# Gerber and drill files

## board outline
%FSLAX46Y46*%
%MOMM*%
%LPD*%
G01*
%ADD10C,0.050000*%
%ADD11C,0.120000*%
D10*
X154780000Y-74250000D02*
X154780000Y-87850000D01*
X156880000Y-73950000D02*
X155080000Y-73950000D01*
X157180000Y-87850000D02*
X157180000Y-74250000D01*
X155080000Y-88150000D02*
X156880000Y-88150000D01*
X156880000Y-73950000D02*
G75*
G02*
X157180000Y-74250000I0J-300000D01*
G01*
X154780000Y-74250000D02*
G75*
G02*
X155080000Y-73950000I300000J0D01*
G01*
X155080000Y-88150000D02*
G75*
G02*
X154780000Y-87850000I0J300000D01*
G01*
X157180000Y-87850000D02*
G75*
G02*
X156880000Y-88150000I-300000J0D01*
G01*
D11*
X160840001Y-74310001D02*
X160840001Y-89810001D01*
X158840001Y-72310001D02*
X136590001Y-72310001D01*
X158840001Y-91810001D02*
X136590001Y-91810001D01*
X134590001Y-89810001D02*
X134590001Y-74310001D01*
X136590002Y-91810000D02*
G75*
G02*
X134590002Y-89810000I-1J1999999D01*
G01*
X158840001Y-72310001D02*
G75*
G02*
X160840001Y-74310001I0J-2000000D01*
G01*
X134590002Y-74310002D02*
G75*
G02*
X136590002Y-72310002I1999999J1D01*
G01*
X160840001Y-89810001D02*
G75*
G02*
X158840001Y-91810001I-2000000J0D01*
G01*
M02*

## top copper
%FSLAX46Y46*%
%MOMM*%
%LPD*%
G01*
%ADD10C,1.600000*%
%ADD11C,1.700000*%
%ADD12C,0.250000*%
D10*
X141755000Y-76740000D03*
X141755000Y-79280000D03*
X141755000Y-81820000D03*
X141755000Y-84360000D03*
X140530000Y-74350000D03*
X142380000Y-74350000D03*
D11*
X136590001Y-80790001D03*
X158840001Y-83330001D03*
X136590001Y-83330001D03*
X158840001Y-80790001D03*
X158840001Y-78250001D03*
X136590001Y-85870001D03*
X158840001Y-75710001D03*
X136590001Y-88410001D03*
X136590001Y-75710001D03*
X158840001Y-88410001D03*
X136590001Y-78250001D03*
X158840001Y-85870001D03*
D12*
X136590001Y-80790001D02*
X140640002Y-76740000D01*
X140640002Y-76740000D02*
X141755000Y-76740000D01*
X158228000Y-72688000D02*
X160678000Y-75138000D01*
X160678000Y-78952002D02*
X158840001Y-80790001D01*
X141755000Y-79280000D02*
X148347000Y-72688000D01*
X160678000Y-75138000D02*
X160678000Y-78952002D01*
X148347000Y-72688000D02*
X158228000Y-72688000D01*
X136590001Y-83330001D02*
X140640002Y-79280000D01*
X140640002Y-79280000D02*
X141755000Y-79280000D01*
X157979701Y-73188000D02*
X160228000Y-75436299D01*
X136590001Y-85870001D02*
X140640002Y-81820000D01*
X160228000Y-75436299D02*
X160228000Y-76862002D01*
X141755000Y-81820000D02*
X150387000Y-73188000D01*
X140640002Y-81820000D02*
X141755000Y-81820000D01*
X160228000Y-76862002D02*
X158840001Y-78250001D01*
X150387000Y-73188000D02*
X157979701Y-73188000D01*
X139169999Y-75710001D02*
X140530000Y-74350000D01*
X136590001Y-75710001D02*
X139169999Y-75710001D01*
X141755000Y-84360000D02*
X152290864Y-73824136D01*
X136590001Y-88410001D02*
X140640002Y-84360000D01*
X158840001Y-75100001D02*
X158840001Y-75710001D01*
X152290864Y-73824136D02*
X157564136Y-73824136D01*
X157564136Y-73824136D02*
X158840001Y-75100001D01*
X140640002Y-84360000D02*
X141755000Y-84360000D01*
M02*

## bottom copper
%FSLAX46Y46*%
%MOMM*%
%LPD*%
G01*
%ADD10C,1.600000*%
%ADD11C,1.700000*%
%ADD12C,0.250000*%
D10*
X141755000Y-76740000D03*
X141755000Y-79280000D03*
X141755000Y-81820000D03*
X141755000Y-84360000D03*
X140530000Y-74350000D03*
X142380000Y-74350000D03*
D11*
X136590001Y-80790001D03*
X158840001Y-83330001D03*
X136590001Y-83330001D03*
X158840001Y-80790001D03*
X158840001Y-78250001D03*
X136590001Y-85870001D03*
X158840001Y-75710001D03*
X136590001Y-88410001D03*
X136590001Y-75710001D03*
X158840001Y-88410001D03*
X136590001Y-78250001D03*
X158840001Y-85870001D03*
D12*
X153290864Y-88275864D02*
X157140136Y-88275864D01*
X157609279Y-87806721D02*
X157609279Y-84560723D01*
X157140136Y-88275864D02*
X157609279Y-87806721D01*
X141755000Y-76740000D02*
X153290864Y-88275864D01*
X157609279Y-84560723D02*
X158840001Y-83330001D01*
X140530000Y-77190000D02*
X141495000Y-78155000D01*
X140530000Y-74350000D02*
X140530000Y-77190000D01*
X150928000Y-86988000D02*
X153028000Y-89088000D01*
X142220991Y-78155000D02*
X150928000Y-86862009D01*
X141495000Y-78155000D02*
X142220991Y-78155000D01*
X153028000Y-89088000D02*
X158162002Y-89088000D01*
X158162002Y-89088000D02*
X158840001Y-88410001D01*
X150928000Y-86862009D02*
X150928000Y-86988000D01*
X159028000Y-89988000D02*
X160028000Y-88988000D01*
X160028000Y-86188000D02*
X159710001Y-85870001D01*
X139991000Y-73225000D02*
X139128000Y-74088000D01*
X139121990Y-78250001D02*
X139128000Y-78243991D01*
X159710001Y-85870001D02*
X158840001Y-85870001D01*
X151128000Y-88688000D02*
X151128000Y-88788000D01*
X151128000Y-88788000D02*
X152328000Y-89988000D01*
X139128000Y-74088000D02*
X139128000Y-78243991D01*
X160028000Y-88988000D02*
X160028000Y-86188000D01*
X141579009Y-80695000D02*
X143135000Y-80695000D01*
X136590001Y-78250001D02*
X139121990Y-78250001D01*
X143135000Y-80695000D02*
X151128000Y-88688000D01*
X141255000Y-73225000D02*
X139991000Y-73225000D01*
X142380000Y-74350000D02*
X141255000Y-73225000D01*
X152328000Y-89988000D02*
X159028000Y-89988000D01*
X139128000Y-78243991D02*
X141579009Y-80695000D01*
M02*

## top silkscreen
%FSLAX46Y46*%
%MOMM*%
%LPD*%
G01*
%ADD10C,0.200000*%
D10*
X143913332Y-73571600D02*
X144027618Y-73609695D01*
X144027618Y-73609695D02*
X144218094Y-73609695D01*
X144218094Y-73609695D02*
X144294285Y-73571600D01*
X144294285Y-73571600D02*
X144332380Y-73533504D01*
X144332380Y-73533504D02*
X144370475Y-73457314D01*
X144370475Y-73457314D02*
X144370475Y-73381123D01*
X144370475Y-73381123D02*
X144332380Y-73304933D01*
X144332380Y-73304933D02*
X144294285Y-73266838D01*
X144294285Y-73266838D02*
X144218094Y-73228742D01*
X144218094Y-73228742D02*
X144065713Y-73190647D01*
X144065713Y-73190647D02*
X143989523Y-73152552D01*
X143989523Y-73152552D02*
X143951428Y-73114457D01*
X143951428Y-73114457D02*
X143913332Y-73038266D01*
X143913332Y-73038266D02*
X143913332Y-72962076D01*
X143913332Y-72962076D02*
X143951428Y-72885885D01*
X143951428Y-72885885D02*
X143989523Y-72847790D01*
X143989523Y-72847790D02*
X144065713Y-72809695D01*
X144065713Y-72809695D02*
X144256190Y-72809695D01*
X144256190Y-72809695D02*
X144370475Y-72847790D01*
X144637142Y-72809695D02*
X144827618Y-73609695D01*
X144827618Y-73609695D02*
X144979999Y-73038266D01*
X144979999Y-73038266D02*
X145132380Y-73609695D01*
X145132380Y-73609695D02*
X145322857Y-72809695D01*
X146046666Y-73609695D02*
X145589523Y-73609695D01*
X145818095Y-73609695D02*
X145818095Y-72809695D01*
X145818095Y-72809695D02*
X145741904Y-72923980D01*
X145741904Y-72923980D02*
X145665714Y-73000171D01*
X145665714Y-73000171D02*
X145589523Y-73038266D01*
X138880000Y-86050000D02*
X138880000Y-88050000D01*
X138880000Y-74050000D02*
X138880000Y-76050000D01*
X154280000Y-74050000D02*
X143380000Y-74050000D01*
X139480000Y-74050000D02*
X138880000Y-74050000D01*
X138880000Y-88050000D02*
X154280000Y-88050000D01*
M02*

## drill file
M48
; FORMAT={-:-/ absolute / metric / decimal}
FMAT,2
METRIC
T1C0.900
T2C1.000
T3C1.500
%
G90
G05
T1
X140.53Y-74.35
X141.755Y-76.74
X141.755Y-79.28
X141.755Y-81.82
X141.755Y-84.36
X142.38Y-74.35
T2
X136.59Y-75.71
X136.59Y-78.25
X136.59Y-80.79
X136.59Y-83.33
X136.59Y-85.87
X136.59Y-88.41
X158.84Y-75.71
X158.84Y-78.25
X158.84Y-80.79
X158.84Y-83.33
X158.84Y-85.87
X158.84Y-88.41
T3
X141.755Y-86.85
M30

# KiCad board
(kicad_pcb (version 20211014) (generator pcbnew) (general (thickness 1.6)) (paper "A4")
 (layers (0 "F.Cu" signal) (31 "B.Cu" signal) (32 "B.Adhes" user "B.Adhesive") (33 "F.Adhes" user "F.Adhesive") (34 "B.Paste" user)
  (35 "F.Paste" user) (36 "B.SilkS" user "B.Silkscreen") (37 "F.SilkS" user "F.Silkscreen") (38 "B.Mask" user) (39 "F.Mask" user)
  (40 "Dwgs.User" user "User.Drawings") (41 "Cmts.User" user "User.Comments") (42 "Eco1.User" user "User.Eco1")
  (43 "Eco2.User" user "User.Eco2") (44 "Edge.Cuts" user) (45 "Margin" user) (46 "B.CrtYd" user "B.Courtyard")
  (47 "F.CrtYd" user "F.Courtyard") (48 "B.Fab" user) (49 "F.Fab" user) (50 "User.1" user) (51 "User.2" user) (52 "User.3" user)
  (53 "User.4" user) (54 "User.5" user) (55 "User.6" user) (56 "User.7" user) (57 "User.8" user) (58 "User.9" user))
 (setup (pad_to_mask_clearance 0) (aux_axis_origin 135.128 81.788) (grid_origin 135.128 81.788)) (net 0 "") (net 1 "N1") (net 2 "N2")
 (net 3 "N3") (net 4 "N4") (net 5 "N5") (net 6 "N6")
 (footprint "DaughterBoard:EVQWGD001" (layer "F.Cu") (at 147.38 80.55)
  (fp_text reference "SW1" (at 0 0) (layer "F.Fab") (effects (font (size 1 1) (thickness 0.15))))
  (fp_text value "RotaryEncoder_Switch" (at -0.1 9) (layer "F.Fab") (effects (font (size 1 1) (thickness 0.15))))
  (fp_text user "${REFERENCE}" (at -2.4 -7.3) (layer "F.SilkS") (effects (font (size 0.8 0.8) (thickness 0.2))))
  (fp_line (start -8.5 5.5) (end -8.5 7.5) (layer "F.SilkS") (width 0.2))
  (fp_line (start -8.5 -6.5) (end -8.5 -4.5) (layer "F.SilkS") (width 0.2))
  (fp_line (start 6.9 -6.5) (end -4 -6.5) (layer "F.SilkS") (width 0.2))
  (fp_line (start -7.9 -6.5) (end -8.5 -6.5) (layer "F.SilkS") (width 0.2))
  (fp_line (start -8.5 7.5) (end 6.9 7.5) (layer "F.SilkS") (width 0.2))
  (fp_line (start 7.4 -6.3) (end 7.4 7.3) (layer "Edge.Cuts") (width 0.05))
  (fp_line (start 9.5 -6.6) (end 7.7 -6.6) (layer "Edge.Cuts") (width 0.05))
  (fp_line (start 9.8 7.3) (end 9.8 -6.3) (layer "Edge.Cuts") (width 0.05))
  (fp_line (start 7.7 7.6) (end 9.5 7.6) (layer "Edge.Cuts") (width 0.05))
  (fp_arc (start 9.5 -6.6) (mid 9.712132 -6.512132) (end 9.8 -6.3) (layer "Edge.Cuts") (width 0.05))
  (fp_arc (start 7.4 -6.3) (mid 7.487868 -6.512132) (end 7.7 -6.6) (layer "Edge.Cuts") (width 0.05))
  (fp_arc (start 7.7 7.6) (mid 7.487868 7.512132) (end 7.4 7.3) (layer "Edge.Cuts") (width 0.05))
  (fp_arc (start 9.8 7.3) (mid 9.712132 7.512132) (end 9.5 7.6) (layer "Edge.Cuts") (width 0.05))
  (pad "" np_thru_hole circle (at -5.625 6.3) (size 1.5 1.5) (drill 1.5) (layers *.Cu *.Mask))
  (pad "A" thru_hole circle (at -5.625 -3.81) (size 1.6 1.6) (drill 0.9) (layers *.Cu *.Mask) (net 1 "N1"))
  (pad "B" thru_hole circle (at -5.625 -1.27) (size 1.6 1.6) (drill 0.9) (layers *.Cu *.Mask) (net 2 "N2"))
  (pad "C" thru_hole circle (at -5.625 1.27) (size 1.6 1.6) (drill 0.9) (layers *.Cu *.Mask) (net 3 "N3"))
  (pad "D" thru_hole circle (at -5.625 3.81) (size 1.6 1.6) (drill 0.9) (layers *.Cu *.Mask) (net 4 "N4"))
  (pad "S1" thru_hole circle (at -6.85 -6.2) (size 1.6 1.6) (drill 0.9) (layers *.Cu *.Mask) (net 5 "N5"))
  (pad "S2" thru_hole circle (at -5 -6.2) (size 1.6 1.6) (drill 0.9) (layers *.Cu *.Mask) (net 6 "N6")))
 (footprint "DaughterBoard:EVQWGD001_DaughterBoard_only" (layer "F.Cu") (at 147.840001 82.060001)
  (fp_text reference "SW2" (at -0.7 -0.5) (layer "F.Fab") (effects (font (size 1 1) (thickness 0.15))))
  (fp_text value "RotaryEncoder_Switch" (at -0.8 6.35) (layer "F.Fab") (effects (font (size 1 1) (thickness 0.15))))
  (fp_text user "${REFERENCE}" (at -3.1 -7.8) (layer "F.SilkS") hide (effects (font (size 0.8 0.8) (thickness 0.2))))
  (fp_line (start 13 -7.75) (end 13 7.75) (layer "Edge.Cuts") (width 0.12))
  (fp_line (start 11 -9.75) (end -11.25 -9.75) (layer "Edge.Cuts") (width 0.12))
  (fp_line (start 11 9.75) (end -11.25 9.75) (layer "Edge.Cuts") (width 0.12))
  (fp_line (start -13.25 7.75) (end -13.25 -7.75) (layer "Edge.Cuts") (width 0.12))
  (fp_arc (start -11.249999 9.749999) (mid -12.664213 9.164213) (end -13.249999 7.749999) (layer "Edge.Cuts") (width 0.12))
  (fp_arc (start 11 -9.75) (mid 12.414214 -9.164214) (end 13 -7.75) (layer "Edge.Cuts") (width 0.12))
  (fp_arc (start -13.249999 -7.749999) (mid -12.664213 -9.164213) (end -11.249999 -9.749999) (layer "Edge.Cuts") (width 0.12))
  (fp_arc (start 13 7.75) (mid 12.414214 9.164214) (end 11 9.75) (layer "Edge.Cuts") (width 0.12))
  (pad "A" thru_hole circle (at -11.25 -1.27) (size 1.7 1.7) (drill 1) (layers *.Cu *.Mask) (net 1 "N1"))
  (pad "A" thru_hole circle (at 11 1.27 180) (size 1.7 1.7) (drill 1) (layers *.Cu *.Mask) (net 1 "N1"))
  (pad "B" thru_hole circle (at -11.25 1.27) (size 1.7 1.7) (drill 1) (layers *.Cu *.Mask) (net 2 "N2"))
  (pad "B" thru_hole circle (at 11 -1.27 180) (size 1.7 1.7) (drill 1) (layers *.Cu *.Mask) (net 2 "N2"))
  (pad "C" thru_hole circle (at 11 -3.81 180) (size 1.7 1.7) (drill 1) (layers *.Cu *.Mask) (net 3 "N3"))
  (pad "C" thru_hole circle (at -11.25 3.81) (size 1.7 1.7) (drill 1) (layers *.Cu *.Mask) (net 3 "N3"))
  (pad "D" thru_hole circle (at 11 -6.35 180) (size 1.7 1.7) (drill 1) (layers *.Cu *.Mask) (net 4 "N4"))
  (pad "D" thru_hole circle (at -11.25 6.35) (size 1.7 1.7) (drill 1) (layers *.Cu *.Mask) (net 4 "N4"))
  (pad "S1" thru_hole circle (at -11.25 -6.35) (size 1.7 1.7) (drill 1) (layers *.Cu *.Mask) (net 5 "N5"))
  (pad "S1" thru_hole circle (at 11 6.35 180) (size 1.7 1.7) (drill 1) (layers *.Cu *.Mask) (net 5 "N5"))
  (pad "S2" thru_hole circle (at -11.25 -3.81) (size 1.7 1.7) (drill 1) (layers *.Cu *.Mask) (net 6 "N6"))
  (pad "S2" thru_hole circle (at 11 3.81 180) (size 1.7 1.7) (drill 1) (layers *.Cu *.Mask) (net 6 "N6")))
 (segment (start 136.590001 80.790001) (end 140.640002 76.74) (width 0.25) (layer "F.Cu") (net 1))
 (segment (start 140.640002 76.74) (end 141.755 76.74) (width 0.25) (layer "F.Cu") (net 1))
 (segment (start 153.290864 88.275864) (end 157.140136 88.275864) (width 0.25) (layer "B.Cu") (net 1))
 (segment (start 157.609279 87.806721) (end 157.609279 84.560723) (width 0.25) (layer "B.Cu") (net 1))
 (segment (start 157.140136 88.275864) (end 157.609279 87.806721) (width 0.25) (layer "B.Cu") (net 1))
 (segment (start 141.755 76.74) (end 153.290864 88.275864) (width 0.25) (layer "B.Cu") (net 1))
 (segment (start 157.609279 84.560723) (end 158.840001 83.330001) (width 0.25) (layer "B.Cu") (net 1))
 (segment (start 158.228 72.688) (end 160.678 75.138) (width 0.25) (layer "F.Cu") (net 2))
 (segment (start 160.678 78.952002) (end 158.840001 80.790001) (width 0.25) (layer "F.Cu") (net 2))
 (segment (start 141.755 79.28) (end 148.347 72.688) (width 0.25) (layer "F.Cu") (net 2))
 (segment (start 160.678 75.138) (end 160.678 78.952002) (width 0.25) (layer "F.Cu") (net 2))
 (segment (start 148.347 72.688) (end 158.228 72.688) (width 0.25) (layer "F.Cu") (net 2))
 (segment (start 136.590001 83.330001) (end 140.640002 79.28) (width 0.25) (layer "F.Cu") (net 2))
 (segment (start 140.640002 79.28) (end 141.755 79.28) (width 0.25) (layer "F.Cu") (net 2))
 (segment (start 157.979701 73.188) (end 160.228 75.436299) (width 0.25) (layer "F.Cu") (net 3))
 (segment (start 136.590001 85.870001) (end 140.640002 81.82) (width 0.25) (layer "F.Cu") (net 3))
 (segment (start 160.228 75.436299) (end 160.228 76.862002) (width 0.25) (layer "F.Cu") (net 3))
 (segment (start 141.755 81.82) (end 150.387 73.188) (width 0.25) (layer "F.Cu") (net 3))
 (segment (start 140.640002 81.82) (end 141.755 81.82) (width 0.25) (layer "F.Cu") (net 3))
 (segment (start 160.228 76.862002) (end 158.840001 78.250001) (width 0.25) (layer "F.Cu") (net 3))
 (segment (start 150.387 73.188) (end 157.979701 73.188) (width 0.25) (layer "F.Cu") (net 3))
 (segment (start 139.169999 75.710001) (end 140.53 74.35) (width 0.25) (layer "F.Cu") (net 5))
 (segment (start 136.590001 75.710001) (end 139.169999 75.710001) (width 0.25) (layer "F.Cu") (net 5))
 (segment (start 140.53 77.19) (end 141.495 78.155) (width 0.25) (layer "B.Cu") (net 5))
 (segment (start 140.53 74.35) (end 140.53 77.19) (width 0.25) (layer "B.Cu") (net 5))
 (segment (start 150.928 86.988) (end 153.028 89.088) (width 0.25) (layer "B.Cu") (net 5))
 (segment (start 142.220991 78.155) (end 150.928 86.862009) (width 0.25) (layer "B.Cu") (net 5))
 (segment (start 141.495 78.155) (end 142.220991 78.155) (width 0.25) (layer "B.Cu") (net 5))
 (segment (start 153.028 89.088) (end 158.162002 89.088) (width 0.25) (layer "B.Cu") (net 5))
 (segment (start 158.162002 89.088) (end 158.840001 88.410001) (width 0.25) (layer "B.Cu") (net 5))
 (segment (start 150.928 86.862009) (end 150.928 86.988) (width 0.25) (layer "B.Cu") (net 5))
 (segment (start 159.028 89.988) (end 160.028 88.988) (width 0.25) (layer "B.Cu") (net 6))
 (segment (start 160.028 86.188) (end 159.710001 85.870001) (width 0.25) (layer "B.Cu") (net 6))
 (segment (start 139.991 73.225) (end 139.128 74.088) (width 0.25) (layer "B.Cu") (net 6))
 (segment (start 139.12199 78.250001) (end 139.128 78.243991) (width 0.25) (layer "B.Cu") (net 6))
 (segment (start 159.710001 85.870001) (end 158.840001 85.870001) (width 0.25) (layer "B.Cu") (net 6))
 (segment (start 151.128 88.688) (end 151.128 88.788) (width 0.25) (layer "B.Cu") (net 6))
 (segment (start 151.128 88.788) (end 152.328 89.988) (width 0.25) (layer "B.Cu") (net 6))
 (segment (start 139.128 74.088) (end 139.128 78.243991) (width 0.25) (layer "B.Cu") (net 6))
 (segment (start 160.028 88.988) (end 160.028 86.188) (width 0.25) (layer "B.Cu") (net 6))
 (segment (start 141.579009 80.695) (end 143.135 80.695) (width 0.25) (layer "B.Cu") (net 6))
 (segment (start 136.590001 78.250001) (end 139.12199 78.250001) (width 0.25) (layer "B.Cu") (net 6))
 (segment (start 143.135 80.695) (end 151.128 88.688) (width 0.25) (layer "B.Cu") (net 6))
 (segment (start 141.255 73.225) (end 139.991 73.225) (width 0.25) (layer "B.Cu") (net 6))
 (segment (start 142.38 74.35) (end 141.255 73.225) (width 0.25) (layer "B.Cu") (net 6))
 (segment (start 152.328 89.988) (end 159.028 89.988) (width 0.25) (layer "B.Cu") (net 6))
 (segment (start 139.128 78.243991) (end 141.579009 80.695) (width 0.25) (layer "B.Cu") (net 6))
 (segment (start 141.755 84.36) (end 152.290864 73.824136) (width 0.25) (layer "F.Cu") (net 4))
 (segment (start 136.590001 88.410001) (end 140.640002 84.36) (width 0.25) (layer "F.Cu") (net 4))
 (segment (start 158.840001 75.100001) (end 158.840001 75.710001) (width 0.25) (layer "F.Cu") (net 4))
 (segment (start 152.290864 73.824136) (end 157.564136 73.824136) (width 0.25) (layer "F.Cu") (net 4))
 (segment (start 157.564136 73.824136) (end 158.840001 75.100001) (width 0.25) (layer "F.Cu") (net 4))
 (segment (start 140.640002 84.36) (end 141.755 84.36) (width 0.25) (layer "F.Cu") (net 4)))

